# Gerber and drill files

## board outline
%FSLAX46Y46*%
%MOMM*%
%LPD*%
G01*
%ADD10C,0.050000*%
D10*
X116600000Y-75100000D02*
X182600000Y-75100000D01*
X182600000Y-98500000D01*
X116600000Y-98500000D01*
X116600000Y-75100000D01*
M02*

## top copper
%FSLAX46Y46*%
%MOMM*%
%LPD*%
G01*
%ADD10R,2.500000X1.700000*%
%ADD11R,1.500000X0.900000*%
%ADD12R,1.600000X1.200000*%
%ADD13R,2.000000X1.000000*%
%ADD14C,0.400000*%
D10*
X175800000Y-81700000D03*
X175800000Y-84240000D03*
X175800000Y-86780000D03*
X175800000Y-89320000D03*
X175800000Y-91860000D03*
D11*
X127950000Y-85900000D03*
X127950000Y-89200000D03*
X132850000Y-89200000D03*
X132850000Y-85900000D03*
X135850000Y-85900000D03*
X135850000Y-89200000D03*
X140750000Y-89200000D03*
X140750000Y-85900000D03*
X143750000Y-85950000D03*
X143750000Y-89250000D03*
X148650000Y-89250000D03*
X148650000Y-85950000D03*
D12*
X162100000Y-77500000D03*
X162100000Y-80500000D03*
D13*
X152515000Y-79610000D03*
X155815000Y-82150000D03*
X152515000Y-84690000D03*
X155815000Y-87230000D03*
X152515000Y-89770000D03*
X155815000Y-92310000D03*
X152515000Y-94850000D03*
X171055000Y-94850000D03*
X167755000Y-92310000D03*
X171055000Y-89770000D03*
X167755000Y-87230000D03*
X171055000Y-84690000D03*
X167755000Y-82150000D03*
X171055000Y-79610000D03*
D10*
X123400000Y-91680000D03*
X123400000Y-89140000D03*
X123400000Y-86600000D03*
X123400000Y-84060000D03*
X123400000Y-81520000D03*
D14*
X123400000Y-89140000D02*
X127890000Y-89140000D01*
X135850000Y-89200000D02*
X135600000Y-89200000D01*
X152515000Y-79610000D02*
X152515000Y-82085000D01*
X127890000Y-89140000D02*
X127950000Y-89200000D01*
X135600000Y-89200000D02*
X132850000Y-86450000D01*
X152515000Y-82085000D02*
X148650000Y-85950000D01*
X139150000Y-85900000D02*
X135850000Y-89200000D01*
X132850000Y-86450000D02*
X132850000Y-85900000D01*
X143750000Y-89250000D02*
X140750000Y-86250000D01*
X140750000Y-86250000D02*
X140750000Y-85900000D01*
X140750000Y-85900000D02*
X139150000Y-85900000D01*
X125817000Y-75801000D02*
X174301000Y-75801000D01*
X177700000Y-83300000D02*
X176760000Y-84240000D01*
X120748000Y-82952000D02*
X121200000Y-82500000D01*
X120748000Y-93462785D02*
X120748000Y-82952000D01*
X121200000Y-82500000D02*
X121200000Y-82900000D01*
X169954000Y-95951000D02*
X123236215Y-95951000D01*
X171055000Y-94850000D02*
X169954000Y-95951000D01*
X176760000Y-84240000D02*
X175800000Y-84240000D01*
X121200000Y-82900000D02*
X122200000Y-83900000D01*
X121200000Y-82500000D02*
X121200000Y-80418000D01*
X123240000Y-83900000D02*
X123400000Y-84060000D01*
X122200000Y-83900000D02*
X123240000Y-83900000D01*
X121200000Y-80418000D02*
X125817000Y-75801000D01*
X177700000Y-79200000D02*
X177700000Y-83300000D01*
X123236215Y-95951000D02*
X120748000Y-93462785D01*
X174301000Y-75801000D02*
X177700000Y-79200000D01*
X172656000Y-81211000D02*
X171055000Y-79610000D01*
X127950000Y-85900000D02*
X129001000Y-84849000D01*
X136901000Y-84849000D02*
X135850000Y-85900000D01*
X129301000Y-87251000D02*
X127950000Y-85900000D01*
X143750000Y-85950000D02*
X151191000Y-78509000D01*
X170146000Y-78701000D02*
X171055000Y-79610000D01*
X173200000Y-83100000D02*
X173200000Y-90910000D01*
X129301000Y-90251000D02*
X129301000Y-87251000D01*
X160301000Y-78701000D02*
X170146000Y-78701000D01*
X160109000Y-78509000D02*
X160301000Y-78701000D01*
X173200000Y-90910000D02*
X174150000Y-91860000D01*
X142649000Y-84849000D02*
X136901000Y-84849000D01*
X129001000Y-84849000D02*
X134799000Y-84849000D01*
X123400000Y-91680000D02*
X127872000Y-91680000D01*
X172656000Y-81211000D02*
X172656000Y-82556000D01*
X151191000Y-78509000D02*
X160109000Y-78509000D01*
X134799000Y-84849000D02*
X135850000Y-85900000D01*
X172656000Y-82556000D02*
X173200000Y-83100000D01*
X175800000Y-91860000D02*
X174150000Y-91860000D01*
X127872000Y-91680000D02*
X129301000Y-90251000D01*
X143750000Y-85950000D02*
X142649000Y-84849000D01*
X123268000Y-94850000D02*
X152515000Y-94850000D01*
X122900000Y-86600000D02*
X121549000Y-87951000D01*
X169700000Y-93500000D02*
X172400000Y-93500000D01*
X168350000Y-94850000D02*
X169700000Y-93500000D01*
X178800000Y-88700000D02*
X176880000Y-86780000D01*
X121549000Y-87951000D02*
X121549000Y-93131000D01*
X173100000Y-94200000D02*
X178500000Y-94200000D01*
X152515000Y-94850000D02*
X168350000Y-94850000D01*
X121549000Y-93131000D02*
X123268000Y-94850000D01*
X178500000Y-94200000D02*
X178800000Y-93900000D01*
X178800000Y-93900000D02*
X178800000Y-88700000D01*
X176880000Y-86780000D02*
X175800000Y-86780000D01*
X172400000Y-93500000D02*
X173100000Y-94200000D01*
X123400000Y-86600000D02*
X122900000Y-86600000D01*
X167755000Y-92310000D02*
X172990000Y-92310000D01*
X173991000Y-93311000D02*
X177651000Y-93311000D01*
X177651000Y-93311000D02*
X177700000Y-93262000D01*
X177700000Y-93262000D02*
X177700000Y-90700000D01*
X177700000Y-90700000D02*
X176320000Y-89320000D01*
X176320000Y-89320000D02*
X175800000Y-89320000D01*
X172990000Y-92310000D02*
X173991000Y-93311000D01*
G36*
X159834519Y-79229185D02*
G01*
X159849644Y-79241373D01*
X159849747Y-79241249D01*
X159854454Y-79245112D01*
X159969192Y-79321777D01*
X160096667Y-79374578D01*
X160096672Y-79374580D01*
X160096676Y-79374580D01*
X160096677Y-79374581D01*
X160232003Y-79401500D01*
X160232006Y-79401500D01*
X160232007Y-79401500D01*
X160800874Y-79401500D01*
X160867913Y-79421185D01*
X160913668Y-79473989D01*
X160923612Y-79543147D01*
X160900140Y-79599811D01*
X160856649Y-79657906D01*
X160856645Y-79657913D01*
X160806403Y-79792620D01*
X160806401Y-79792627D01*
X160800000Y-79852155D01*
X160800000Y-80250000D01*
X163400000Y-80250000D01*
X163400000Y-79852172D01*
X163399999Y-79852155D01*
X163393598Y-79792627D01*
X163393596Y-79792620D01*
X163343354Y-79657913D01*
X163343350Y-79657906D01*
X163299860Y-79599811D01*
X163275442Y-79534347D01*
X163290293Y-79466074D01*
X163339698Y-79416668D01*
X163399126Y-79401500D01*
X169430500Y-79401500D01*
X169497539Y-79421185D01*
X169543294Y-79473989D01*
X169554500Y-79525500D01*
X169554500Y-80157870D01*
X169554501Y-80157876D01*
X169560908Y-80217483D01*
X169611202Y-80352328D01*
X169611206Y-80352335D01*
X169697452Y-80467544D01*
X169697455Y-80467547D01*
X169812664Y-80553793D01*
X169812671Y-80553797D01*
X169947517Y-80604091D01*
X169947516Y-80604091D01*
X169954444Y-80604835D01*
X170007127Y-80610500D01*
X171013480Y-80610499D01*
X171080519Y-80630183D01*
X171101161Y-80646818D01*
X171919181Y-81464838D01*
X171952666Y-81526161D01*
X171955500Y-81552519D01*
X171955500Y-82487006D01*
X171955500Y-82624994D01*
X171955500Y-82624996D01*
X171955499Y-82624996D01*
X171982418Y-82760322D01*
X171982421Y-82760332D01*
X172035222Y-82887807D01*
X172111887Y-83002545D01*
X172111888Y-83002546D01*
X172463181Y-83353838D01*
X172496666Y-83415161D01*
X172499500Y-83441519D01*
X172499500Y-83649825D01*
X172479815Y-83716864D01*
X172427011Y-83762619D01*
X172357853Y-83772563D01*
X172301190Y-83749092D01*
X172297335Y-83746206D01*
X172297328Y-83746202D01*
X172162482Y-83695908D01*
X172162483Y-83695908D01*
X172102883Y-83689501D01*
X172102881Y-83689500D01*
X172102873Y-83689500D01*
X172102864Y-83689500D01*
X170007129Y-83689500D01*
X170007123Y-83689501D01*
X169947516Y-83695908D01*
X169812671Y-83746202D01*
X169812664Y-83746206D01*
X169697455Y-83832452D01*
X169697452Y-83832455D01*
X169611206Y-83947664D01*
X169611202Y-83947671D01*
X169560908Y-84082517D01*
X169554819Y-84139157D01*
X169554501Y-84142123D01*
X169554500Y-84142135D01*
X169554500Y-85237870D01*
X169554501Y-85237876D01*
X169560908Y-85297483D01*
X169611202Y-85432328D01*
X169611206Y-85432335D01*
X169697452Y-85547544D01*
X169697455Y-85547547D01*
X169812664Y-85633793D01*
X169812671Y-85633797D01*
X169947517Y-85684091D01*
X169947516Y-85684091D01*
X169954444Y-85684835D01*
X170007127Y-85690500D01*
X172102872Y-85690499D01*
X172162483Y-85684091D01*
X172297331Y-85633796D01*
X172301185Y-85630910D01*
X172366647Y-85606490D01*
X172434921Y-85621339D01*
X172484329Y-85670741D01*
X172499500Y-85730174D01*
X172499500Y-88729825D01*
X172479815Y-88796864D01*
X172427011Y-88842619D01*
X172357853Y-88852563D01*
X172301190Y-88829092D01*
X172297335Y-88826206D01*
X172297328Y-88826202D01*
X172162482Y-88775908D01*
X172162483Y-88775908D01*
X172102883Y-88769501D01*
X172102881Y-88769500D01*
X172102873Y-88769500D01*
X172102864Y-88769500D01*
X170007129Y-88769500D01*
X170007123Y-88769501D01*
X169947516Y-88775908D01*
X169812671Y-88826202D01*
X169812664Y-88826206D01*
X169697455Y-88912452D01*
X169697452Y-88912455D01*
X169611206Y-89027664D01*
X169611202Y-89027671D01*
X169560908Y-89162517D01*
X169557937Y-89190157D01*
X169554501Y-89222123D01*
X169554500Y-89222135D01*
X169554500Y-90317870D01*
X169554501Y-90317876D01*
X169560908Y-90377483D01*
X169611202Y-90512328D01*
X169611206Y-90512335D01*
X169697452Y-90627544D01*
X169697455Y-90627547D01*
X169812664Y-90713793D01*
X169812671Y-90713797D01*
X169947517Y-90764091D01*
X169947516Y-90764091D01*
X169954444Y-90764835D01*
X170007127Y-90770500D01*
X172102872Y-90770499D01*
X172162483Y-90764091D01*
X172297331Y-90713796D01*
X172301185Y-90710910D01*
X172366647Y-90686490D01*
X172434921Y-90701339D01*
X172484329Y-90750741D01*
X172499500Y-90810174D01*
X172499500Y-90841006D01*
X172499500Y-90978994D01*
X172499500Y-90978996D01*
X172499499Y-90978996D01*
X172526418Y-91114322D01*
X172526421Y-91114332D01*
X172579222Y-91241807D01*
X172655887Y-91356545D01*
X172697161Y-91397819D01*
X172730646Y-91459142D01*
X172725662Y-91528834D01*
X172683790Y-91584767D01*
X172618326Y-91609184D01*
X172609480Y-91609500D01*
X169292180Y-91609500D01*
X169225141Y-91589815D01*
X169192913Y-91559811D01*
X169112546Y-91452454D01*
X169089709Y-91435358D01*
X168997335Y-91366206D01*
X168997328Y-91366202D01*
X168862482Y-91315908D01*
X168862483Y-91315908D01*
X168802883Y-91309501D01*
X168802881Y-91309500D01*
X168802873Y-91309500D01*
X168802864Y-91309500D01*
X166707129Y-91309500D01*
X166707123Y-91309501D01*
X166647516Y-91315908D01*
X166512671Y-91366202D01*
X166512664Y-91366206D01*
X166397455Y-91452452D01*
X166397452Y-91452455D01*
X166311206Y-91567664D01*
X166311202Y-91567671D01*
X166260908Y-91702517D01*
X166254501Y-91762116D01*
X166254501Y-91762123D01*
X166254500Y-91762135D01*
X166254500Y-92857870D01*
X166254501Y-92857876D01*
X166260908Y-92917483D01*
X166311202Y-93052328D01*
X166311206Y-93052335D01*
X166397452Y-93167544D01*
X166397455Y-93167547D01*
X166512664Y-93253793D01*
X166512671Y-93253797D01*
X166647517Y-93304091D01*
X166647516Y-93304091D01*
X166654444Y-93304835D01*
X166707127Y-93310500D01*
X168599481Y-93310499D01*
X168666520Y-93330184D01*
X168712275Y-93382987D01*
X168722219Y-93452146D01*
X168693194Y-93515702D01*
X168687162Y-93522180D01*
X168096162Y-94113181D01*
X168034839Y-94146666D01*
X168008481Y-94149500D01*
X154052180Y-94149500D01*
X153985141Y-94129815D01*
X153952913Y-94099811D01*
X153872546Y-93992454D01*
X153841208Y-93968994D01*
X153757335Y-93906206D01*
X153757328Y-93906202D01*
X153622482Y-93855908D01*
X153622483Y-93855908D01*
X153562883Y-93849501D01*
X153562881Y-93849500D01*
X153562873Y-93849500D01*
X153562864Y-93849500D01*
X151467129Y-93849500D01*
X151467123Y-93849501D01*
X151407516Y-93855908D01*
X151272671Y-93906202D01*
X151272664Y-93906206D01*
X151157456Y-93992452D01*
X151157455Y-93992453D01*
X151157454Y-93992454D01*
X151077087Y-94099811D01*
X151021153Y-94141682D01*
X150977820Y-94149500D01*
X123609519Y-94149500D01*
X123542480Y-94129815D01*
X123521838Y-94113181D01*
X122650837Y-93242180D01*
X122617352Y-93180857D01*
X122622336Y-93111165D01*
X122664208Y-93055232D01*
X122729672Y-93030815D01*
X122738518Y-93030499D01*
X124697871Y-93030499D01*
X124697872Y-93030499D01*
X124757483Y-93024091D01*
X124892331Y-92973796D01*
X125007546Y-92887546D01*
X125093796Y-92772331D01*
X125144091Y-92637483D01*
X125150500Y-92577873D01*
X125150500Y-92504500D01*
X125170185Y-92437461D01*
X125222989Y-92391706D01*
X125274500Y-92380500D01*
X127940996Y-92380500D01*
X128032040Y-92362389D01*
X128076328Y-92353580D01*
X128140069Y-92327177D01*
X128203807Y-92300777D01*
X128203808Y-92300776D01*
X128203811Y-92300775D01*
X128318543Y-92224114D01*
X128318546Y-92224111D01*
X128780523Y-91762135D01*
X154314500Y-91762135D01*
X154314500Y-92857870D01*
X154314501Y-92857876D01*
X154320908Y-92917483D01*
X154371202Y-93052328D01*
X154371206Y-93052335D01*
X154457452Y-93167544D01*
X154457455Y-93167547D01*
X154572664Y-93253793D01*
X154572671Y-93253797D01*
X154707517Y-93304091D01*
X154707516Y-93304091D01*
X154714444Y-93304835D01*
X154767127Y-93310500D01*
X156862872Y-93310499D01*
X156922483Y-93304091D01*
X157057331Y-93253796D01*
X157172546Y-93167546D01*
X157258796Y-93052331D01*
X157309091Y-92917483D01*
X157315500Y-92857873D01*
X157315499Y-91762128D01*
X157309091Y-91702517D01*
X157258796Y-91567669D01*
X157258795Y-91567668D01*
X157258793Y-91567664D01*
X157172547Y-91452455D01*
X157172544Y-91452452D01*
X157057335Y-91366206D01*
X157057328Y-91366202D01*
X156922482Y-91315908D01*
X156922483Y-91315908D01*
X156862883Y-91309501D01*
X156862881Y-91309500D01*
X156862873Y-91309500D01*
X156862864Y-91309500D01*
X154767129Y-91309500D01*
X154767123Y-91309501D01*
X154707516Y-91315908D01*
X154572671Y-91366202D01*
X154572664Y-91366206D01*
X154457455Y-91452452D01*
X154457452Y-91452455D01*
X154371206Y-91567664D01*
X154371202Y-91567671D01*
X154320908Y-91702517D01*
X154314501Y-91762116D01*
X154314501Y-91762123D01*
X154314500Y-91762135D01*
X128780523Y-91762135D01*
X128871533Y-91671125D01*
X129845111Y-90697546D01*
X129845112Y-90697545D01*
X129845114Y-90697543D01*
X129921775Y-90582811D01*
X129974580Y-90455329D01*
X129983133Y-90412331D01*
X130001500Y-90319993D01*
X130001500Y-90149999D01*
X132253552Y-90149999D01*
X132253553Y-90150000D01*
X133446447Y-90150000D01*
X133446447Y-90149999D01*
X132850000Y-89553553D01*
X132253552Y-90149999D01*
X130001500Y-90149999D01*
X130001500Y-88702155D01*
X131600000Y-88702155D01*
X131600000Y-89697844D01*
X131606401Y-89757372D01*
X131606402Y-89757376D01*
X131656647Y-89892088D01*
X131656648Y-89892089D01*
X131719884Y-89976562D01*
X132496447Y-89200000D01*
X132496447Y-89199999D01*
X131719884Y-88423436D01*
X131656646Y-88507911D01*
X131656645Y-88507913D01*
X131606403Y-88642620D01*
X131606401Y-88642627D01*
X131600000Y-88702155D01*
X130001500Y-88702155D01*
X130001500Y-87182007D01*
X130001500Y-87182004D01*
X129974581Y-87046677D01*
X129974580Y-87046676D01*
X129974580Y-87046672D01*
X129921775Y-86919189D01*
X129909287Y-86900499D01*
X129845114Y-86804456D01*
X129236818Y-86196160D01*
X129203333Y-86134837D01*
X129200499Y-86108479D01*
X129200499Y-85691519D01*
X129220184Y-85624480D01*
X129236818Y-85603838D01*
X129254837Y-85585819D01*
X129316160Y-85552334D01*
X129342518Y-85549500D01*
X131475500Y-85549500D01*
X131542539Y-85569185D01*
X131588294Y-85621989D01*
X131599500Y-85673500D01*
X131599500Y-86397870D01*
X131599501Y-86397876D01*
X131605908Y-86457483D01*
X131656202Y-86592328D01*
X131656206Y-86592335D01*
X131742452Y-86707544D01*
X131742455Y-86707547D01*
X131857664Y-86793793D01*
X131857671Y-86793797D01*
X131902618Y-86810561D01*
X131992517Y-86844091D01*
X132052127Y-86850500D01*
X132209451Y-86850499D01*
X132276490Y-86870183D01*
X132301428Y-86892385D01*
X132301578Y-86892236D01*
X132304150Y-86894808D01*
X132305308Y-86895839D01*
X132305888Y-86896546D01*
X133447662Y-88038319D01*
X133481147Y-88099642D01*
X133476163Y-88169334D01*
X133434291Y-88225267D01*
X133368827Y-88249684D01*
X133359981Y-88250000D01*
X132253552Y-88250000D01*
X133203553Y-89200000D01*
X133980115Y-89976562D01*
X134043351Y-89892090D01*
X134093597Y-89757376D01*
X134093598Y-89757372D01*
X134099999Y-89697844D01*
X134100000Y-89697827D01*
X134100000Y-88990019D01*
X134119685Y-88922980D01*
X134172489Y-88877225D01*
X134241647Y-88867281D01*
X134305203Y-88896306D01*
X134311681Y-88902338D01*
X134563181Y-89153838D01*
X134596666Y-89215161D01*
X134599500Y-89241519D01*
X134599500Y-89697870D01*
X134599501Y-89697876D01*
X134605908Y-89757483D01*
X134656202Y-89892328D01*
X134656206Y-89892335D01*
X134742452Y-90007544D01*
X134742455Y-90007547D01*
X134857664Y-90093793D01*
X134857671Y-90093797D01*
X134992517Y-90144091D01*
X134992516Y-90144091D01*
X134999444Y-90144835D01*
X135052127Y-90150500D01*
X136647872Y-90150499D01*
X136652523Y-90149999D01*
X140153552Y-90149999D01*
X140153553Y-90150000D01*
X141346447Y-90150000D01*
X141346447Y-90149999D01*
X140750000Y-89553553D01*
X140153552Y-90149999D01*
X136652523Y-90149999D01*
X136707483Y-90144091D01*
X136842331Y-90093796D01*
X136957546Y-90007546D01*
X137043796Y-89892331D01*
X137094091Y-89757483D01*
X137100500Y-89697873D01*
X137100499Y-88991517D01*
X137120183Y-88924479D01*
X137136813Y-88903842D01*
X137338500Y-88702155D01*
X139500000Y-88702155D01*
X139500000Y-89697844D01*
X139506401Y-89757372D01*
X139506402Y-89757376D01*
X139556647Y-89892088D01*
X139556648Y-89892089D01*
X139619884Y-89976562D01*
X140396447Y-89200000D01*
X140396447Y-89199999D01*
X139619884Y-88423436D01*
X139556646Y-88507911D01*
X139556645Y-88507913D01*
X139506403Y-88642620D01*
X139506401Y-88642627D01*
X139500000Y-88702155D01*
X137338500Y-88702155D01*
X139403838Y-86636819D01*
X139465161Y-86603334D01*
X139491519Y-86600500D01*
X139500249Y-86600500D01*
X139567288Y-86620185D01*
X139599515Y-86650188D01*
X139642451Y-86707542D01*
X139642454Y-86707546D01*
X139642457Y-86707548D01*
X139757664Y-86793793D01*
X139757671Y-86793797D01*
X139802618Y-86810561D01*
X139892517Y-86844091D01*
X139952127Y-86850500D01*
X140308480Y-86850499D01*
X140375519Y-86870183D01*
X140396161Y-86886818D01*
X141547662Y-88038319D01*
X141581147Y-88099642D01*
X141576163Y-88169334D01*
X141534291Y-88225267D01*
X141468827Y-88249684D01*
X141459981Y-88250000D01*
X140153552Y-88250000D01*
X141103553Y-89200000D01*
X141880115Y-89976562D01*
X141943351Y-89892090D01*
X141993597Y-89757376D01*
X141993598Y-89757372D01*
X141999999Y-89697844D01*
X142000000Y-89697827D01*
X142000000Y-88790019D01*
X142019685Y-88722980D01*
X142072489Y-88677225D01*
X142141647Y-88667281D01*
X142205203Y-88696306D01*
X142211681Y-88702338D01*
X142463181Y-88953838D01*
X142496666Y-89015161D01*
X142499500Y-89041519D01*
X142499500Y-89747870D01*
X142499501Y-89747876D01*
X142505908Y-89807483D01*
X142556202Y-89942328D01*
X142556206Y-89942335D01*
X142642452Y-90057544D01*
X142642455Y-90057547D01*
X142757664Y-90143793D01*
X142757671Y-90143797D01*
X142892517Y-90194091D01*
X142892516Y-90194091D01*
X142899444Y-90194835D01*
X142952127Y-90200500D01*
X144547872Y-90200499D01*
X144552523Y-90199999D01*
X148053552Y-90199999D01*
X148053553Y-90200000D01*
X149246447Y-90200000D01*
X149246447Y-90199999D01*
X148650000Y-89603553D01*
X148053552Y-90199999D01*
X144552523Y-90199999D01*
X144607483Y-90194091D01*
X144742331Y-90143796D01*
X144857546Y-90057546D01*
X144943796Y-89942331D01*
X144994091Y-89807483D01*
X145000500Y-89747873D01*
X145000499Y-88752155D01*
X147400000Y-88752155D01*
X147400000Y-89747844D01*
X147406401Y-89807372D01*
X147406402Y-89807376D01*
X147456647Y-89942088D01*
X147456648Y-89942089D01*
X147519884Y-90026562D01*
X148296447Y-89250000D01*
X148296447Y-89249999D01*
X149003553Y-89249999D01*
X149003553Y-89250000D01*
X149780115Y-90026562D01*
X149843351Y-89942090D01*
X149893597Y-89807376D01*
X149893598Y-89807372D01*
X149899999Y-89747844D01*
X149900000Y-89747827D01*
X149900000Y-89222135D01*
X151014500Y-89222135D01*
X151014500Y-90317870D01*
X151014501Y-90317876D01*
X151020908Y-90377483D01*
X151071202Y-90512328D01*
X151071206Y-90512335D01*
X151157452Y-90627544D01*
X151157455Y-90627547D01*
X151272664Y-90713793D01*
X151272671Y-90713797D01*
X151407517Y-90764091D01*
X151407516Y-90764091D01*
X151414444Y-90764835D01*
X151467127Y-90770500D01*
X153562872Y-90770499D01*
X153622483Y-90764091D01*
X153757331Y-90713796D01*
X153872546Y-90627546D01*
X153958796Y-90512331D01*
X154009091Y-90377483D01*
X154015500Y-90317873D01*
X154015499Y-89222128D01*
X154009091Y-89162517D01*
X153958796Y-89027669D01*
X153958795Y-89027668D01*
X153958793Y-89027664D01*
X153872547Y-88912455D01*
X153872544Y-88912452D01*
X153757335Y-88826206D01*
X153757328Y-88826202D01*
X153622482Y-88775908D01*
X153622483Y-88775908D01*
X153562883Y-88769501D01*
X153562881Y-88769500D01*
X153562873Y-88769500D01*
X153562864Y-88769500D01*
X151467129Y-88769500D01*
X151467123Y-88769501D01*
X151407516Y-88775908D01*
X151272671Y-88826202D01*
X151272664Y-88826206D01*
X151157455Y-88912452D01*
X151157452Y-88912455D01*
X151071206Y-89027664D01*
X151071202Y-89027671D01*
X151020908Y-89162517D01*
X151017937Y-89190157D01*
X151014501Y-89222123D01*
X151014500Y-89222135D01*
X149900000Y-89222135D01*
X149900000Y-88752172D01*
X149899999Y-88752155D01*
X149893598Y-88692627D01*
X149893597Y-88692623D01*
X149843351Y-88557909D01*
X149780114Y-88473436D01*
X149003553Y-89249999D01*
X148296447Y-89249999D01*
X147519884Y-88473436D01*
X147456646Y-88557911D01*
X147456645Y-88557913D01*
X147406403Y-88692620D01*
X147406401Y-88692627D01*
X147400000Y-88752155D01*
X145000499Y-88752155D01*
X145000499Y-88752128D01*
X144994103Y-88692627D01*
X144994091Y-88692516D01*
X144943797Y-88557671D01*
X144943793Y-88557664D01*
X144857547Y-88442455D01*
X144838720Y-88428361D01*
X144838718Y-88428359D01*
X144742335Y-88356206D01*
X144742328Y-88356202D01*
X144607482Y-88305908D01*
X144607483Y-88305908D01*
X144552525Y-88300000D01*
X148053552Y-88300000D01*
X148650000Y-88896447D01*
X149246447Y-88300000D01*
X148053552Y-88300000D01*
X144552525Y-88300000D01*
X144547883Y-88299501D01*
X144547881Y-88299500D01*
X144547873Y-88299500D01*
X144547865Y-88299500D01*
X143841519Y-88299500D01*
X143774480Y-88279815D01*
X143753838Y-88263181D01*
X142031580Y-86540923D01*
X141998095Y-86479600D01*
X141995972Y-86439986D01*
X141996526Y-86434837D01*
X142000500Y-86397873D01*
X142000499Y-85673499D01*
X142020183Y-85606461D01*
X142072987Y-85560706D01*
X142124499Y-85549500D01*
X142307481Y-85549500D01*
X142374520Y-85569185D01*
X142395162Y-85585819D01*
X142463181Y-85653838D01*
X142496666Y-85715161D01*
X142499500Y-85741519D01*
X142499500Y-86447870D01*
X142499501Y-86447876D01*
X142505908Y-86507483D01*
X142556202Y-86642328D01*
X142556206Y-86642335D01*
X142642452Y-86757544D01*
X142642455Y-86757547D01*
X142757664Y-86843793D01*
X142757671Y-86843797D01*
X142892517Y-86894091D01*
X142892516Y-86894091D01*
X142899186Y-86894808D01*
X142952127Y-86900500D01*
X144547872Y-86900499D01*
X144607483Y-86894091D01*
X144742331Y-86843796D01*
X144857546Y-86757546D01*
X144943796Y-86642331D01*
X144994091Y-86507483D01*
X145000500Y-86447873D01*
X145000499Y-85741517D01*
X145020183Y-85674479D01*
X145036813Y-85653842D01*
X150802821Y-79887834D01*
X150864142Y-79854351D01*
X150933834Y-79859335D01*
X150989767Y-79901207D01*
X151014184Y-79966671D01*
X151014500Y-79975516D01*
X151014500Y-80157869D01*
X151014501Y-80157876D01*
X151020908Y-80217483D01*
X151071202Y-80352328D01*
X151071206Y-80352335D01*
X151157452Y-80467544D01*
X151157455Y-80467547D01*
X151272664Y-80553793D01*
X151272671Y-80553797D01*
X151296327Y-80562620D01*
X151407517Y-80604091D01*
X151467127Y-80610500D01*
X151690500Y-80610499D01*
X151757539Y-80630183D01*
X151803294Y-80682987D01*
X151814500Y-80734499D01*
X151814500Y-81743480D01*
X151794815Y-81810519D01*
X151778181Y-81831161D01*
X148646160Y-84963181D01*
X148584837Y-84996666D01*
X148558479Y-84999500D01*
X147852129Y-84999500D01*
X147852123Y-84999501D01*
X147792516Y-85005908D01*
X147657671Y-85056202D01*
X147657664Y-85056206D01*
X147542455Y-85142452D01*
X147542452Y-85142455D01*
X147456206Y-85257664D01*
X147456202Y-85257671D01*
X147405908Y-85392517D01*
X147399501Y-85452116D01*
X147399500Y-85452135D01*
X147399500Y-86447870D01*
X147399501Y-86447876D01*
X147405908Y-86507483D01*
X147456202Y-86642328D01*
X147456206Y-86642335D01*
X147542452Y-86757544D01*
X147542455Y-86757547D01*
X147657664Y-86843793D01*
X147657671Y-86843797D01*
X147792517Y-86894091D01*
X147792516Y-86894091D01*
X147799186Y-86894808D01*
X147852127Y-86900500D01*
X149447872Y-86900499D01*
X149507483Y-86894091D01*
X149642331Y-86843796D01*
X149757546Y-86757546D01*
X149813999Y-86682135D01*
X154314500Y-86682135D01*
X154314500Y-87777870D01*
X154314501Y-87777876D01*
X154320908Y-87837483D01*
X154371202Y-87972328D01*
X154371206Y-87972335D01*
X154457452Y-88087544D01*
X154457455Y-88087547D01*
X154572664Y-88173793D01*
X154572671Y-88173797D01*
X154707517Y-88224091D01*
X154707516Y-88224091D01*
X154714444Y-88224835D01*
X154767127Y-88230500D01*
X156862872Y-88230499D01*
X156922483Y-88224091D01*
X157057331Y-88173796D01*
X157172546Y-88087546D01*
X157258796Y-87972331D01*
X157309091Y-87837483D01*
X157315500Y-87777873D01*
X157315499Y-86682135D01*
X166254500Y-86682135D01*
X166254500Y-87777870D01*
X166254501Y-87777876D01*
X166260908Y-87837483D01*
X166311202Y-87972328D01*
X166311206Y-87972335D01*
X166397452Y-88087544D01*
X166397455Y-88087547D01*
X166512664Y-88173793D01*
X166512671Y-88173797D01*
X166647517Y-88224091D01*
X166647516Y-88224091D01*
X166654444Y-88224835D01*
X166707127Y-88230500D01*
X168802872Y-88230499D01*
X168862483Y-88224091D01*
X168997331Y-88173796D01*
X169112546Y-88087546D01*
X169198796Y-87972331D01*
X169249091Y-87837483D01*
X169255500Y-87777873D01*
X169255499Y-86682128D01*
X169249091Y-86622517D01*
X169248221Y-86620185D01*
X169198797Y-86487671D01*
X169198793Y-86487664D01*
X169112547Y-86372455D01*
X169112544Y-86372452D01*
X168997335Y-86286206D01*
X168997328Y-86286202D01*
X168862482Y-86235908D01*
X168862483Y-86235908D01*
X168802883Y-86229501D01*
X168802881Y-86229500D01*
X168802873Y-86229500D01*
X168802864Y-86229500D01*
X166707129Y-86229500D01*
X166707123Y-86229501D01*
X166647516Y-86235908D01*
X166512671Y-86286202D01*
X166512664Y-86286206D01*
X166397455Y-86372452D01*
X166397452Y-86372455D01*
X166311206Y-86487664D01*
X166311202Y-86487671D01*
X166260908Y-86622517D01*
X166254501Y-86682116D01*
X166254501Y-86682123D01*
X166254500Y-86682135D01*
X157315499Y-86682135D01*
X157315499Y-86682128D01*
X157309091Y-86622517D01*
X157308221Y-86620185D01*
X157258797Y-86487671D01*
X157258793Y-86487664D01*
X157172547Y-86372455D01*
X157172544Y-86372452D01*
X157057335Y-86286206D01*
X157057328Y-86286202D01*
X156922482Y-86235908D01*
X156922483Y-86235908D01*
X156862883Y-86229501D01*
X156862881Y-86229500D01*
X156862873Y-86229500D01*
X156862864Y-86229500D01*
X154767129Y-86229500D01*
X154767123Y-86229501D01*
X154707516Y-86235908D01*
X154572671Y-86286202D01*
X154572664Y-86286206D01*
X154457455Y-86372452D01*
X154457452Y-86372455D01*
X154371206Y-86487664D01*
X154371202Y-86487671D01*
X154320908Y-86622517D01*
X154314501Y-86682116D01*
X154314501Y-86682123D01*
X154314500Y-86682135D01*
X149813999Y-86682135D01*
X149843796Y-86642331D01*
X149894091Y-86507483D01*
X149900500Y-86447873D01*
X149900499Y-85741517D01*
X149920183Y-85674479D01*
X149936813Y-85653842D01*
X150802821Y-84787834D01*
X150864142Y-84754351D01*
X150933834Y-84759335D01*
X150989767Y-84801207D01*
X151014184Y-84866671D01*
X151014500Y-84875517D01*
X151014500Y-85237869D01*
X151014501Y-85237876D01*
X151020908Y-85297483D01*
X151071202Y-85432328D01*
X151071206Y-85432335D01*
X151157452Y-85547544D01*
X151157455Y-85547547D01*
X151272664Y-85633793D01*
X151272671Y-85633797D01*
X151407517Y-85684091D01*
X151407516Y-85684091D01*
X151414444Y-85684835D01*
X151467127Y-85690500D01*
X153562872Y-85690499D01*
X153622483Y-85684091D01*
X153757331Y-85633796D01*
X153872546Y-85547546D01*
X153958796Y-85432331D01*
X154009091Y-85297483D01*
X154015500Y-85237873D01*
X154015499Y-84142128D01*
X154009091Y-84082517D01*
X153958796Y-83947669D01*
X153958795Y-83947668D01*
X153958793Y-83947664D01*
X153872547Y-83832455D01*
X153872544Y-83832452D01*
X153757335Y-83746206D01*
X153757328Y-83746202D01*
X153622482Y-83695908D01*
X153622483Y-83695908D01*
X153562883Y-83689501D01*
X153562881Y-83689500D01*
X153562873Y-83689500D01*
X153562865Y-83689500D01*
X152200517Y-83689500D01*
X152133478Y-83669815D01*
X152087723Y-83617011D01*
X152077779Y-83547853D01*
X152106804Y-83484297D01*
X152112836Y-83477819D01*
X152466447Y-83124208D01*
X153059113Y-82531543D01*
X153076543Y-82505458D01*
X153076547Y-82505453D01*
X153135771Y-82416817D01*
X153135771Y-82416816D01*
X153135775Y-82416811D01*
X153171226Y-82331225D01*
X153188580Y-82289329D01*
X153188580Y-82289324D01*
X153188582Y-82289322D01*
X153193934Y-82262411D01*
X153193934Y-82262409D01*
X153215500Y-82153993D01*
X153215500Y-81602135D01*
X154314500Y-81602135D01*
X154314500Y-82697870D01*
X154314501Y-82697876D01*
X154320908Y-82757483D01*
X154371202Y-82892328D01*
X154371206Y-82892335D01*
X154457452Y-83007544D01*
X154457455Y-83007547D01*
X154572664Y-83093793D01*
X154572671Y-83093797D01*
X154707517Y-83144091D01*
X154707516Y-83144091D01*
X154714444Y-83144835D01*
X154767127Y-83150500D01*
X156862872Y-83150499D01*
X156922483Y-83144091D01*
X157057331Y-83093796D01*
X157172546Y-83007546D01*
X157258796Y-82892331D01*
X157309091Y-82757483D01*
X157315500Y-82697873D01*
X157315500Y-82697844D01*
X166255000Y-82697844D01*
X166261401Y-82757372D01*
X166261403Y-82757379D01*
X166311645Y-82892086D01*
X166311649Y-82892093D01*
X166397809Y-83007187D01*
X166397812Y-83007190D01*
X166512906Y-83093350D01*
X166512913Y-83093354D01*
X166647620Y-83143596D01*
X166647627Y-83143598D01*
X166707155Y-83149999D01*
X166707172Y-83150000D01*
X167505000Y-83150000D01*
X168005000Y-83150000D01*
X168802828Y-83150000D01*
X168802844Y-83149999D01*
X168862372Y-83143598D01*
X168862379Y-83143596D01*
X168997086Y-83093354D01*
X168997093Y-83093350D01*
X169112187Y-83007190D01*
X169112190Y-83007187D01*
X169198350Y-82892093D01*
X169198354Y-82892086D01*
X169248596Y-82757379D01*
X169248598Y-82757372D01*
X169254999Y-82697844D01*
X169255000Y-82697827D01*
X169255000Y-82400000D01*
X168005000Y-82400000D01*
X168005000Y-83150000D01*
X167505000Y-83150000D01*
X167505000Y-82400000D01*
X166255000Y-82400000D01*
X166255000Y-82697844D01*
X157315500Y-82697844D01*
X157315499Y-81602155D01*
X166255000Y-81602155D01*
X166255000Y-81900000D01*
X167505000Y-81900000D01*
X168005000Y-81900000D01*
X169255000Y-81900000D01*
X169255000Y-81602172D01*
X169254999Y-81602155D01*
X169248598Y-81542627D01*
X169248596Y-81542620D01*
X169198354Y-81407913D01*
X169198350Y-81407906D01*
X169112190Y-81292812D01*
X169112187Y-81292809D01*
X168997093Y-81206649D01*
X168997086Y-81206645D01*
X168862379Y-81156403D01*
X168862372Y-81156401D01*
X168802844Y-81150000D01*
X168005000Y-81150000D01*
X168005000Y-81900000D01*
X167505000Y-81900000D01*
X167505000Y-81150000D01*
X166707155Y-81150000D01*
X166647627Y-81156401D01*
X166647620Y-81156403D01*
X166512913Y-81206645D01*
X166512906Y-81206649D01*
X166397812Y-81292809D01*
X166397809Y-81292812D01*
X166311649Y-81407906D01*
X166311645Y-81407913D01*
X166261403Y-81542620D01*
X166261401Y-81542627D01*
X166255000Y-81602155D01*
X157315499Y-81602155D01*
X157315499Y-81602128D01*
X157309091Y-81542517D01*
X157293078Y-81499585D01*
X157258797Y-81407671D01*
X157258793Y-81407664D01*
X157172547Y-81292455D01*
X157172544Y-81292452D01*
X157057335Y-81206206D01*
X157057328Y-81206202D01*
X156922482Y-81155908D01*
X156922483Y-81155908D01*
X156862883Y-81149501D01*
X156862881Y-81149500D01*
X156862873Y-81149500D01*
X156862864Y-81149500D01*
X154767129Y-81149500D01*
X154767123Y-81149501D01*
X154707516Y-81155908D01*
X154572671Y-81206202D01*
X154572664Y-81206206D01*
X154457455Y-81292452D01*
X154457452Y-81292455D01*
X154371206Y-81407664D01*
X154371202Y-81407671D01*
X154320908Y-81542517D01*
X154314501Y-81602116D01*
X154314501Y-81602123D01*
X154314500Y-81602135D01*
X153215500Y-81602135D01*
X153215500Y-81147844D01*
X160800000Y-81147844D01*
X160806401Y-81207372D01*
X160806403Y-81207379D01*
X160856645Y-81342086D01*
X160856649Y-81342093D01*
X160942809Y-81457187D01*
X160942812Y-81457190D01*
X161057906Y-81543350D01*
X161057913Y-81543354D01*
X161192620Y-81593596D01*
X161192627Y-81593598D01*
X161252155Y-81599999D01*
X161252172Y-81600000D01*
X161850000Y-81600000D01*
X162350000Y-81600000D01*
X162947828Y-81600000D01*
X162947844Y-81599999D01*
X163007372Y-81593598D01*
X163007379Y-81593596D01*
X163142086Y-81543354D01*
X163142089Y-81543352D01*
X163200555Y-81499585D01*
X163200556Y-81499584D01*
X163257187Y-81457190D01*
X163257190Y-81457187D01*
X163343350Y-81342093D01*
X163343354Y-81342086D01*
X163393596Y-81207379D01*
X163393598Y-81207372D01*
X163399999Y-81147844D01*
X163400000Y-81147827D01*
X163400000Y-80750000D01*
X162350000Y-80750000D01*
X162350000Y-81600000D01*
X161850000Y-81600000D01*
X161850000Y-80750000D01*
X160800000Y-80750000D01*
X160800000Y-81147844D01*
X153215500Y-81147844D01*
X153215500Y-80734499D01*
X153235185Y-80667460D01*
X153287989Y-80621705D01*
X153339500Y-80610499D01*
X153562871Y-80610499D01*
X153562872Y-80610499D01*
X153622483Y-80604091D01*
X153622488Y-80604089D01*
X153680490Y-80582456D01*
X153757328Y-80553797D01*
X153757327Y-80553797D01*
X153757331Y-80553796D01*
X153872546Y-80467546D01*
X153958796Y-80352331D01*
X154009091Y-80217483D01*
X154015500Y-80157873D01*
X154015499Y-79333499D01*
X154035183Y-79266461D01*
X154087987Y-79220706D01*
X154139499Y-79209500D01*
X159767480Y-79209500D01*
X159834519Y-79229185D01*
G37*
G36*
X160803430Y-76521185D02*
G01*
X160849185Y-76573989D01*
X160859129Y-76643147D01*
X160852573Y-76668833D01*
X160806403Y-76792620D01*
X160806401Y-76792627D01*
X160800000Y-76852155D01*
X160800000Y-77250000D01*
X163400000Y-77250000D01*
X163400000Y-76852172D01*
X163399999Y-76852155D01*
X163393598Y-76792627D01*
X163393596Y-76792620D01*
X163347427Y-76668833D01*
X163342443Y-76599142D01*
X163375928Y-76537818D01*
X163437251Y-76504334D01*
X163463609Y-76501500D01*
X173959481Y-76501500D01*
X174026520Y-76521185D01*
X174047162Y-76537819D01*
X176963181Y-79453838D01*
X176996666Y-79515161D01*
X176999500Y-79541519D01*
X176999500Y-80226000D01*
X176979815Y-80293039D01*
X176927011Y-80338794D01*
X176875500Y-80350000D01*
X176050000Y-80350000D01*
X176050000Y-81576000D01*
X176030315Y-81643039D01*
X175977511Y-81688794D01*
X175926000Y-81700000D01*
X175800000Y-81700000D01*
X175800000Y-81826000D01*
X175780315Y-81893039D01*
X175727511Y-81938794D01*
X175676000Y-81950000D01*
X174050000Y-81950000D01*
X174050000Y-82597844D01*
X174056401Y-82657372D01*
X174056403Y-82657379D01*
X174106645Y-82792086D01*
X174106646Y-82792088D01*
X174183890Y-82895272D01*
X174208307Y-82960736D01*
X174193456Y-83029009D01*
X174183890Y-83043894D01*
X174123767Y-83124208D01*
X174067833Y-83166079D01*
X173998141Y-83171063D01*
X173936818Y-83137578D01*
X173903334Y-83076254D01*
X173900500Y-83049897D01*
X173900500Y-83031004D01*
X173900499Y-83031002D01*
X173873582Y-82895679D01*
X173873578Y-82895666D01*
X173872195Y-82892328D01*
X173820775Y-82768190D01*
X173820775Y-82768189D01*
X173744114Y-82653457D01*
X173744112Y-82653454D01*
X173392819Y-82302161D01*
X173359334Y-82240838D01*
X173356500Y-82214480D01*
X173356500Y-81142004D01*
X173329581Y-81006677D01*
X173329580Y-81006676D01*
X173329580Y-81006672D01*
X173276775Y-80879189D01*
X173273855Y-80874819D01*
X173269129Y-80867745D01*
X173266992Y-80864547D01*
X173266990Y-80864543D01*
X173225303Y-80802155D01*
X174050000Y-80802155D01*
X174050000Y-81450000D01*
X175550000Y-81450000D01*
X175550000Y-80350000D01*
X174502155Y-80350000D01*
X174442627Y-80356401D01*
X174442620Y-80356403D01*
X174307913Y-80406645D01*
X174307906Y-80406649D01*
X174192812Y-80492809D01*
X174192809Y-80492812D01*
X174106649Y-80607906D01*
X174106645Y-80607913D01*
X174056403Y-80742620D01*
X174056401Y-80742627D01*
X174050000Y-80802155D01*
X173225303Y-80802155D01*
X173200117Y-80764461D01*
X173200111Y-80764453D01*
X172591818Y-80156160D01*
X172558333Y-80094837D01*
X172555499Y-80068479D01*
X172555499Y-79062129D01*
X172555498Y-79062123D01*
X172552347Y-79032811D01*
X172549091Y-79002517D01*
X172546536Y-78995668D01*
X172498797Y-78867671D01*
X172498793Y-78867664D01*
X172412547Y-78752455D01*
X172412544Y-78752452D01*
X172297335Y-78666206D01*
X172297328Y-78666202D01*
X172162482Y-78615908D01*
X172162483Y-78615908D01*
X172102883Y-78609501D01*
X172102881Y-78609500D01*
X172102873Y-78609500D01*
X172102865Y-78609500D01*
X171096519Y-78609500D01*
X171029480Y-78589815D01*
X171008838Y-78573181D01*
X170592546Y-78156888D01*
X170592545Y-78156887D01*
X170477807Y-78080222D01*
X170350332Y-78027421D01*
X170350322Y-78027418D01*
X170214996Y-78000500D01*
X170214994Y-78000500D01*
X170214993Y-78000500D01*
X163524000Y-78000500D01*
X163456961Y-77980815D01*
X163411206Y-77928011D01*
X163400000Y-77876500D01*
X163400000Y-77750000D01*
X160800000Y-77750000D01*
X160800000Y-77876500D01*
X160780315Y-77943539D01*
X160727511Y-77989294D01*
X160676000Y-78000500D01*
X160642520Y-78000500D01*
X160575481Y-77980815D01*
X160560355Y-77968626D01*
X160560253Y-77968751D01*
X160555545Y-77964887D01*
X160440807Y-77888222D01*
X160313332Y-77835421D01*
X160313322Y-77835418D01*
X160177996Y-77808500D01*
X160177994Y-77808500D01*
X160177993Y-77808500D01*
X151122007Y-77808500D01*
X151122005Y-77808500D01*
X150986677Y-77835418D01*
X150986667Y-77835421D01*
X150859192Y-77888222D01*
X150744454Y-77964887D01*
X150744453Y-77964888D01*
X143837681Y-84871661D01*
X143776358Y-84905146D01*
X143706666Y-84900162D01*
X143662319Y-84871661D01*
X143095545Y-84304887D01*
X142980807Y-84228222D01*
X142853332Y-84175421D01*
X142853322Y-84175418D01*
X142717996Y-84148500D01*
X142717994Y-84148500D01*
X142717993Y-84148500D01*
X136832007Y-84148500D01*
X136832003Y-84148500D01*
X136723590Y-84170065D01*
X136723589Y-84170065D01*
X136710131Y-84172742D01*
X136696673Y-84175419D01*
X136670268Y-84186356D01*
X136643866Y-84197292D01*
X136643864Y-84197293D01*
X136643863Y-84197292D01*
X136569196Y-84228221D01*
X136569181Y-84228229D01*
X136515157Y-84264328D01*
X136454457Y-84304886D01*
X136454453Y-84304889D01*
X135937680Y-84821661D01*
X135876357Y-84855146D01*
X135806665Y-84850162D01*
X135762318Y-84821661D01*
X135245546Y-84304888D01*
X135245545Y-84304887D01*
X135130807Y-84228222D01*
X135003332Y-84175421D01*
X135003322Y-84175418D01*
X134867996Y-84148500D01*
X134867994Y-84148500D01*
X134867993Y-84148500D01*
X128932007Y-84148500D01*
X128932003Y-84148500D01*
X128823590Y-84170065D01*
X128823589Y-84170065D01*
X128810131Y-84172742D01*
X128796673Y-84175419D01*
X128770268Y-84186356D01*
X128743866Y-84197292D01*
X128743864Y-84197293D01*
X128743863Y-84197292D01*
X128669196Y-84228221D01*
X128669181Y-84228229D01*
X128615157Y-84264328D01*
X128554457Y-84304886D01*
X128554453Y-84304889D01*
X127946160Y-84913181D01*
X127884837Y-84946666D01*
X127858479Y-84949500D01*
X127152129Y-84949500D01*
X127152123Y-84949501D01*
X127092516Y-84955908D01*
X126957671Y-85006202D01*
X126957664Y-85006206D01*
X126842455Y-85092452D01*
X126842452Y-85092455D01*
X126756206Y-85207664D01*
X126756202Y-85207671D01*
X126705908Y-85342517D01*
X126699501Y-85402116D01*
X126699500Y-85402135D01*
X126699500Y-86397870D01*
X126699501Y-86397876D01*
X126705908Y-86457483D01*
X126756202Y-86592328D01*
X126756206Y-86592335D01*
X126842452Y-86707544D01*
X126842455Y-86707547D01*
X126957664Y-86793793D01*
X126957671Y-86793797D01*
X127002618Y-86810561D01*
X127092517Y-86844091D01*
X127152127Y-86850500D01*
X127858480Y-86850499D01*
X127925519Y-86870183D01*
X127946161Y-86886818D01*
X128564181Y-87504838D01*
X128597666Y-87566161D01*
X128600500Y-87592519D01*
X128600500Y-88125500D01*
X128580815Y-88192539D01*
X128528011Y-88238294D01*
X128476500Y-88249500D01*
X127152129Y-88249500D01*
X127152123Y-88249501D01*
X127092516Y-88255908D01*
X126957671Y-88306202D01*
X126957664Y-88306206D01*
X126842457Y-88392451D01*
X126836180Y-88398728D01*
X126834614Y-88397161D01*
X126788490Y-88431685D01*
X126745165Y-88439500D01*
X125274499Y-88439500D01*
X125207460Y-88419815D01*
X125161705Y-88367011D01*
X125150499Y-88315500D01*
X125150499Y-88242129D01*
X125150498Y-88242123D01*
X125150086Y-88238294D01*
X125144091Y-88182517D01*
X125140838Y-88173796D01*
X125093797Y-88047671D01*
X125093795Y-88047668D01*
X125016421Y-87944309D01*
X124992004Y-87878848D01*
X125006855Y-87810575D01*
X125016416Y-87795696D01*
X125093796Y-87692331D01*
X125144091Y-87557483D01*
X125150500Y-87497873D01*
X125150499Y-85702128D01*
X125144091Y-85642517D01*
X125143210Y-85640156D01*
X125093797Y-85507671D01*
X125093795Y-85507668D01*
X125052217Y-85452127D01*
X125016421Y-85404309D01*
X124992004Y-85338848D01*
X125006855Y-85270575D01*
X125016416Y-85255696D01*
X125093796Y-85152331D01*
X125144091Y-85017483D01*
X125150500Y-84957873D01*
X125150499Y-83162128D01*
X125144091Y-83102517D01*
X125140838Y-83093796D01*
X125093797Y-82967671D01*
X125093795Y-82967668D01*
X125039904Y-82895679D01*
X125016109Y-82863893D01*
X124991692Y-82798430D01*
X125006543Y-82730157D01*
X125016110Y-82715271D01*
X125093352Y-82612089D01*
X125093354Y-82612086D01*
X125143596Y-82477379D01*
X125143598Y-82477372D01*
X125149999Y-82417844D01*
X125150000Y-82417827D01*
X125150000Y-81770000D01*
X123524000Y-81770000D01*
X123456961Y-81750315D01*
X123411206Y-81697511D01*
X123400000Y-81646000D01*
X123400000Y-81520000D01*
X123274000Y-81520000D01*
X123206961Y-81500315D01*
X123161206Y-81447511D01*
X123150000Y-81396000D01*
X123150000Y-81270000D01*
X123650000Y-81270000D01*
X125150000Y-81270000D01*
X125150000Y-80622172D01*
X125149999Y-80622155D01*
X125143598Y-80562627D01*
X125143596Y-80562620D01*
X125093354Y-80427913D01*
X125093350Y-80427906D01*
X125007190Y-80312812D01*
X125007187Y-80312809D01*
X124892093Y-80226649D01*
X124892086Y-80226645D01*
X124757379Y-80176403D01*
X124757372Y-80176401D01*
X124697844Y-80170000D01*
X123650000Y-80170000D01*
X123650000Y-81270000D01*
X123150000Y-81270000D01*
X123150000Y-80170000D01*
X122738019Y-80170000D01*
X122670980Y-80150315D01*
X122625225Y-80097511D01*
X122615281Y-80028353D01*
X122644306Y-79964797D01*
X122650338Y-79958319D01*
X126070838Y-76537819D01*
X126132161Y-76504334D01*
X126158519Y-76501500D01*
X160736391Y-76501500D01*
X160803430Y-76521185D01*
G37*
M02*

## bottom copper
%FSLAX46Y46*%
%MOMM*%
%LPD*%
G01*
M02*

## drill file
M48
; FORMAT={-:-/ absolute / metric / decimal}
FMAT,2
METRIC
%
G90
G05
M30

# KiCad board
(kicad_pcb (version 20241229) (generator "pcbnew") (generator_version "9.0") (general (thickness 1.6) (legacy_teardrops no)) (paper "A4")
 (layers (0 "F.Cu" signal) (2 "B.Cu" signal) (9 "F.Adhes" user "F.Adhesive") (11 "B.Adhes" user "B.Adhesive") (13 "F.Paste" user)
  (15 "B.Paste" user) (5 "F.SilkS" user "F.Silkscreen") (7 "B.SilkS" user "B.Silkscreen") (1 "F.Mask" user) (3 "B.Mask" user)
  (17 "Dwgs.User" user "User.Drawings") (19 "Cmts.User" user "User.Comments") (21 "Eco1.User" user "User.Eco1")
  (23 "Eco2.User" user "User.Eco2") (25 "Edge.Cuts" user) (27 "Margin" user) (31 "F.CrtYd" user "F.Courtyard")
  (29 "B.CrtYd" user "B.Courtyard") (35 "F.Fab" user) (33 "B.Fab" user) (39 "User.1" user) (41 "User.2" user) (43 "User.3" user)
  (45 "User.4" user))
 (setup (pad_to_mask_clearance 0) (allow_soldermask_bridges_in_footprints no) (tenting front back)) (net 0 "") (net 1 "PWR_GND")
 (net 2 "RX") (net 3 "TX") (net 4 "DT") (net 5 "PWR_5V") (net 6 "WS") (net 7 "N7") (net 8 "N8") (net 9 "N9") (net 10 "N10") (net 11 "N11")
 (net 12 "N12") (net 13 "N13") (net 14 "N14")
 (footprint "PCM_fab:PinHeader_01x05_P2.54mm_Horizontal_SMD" (layer "F.Cu") (at 175.8 81.7)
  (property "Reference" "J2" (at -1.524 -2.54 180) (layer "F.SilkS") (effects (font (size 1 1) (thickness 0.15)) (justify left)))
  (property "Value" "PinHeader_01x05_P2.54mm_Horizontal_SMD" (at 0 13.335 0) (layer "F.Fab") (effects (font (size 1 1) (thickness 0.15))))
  (pad "1" smd rect (at 0 0) (size 2.5 1.7) (layers "F.Cu" "F.Mask" "F.Paste") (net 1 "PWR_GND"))
  (pad "2" smd rect (at 0 2.54) (size 2.5 1.7) (layers "F.Cu" "F.Mask" "F.Paste") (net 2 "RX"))
  (pad "3" smd rect (at 0 5.08) (size 2.5 1.7) (layers "F.Cu" "F.Mask" "F.Paste") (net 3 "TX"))
  (pad "4" smd rect (at 0 7.62) (size 2.5 1.7) (layers "F.Cu" "F.Mask" "F.Paste") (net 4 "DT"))
  (pad "5" smd rect (at 0 10.16) (size 2.5 1.7) (layers "F.Cu" "F.Mask" "F.Paste") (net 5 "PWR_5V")))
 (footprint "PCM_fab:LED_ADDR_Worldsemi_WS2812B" (layer "F.Cu") (at 130.4 87.55)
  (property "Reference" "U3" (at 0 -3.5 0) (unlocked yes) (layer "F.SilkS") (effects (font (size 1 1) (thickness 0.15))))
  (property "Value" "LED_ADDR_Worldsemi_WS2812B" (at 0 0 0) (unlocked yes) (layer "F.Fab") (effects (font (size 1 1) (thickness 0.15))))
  (pad "1" smd rect (at -2.45 -1.65) (size 1.5 0.9) (layers "F.Cu" "F.Mask" "F.Paste") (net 5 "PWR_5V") (thermal_bridge_angle 45))
  (pad "2" smd rect (at -2.45 1.65) (size 1.5 0.9) (layers "F.Cu" "F.Mask" "F.Paste") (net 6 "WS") (thermal_bridge_angle 45))
  (pad "3" smd rect (at 2.45 1.65) (size 1.5 0.9) (layers "F.Cu" "F.Mask" "F.Paste") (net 1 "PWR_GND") (thermal_bridge_angle 45))
  (pad "4" smd rect (at 2.45 -1.65) (size 1.5 0.9) (layers "F.Cu" "F.Mask" "F.Paste") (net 6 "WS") (thermal_bridge_angle 45)))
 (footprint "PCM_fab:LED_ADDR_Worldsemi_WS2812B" (layer "F.Cu") (at 138.3 87.55)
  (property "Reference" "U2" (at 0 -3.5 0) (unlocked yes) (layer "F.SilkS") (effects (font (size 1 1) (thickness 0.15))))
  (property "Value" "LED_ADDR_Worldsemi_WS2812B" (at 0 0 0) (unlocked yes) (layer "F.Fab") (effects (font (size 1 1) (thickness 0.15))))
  (pad "1" smd rect (at -2.45 -1.65) (size 1.5 0.9) (layers "F.Cu" "F.Mask" "F.Paste") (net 5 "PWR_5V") (thermal_bridge_angle 45))
  (pad "2" smd rect (at -2.45 1.65) (size 1.5 0.9) (layers "F.Cu" "F.Mask" "F.Paste") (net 6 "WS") (thermal_bridge_angle 45))
  (pad "3" smd rect (at 2.45 1.65) (size 1.5 0.9) (layers "F.Cu" "F.Mask" "F.Paste") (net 1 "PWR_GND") (thermal_bridge_angle 45))
  (pad "4" smd rect (at 2.45 -1.65) (size 1.5 0.9) (layers "F.Cu" "F.Mask" "F.Paste") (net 6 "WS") (thermal_bridge_angle 45)))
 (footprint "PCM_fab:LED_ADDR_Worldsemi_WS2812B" (layer "F.Cu") (at 146.2 87.6)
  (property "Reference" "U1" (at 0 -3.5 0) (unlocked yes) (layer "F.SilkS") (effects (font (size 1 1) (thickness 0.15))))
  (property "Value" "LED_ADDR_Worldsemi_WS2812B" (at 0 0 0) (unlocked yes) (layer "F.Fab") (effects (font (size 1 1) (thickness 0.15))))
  (pad "1" smd rect (at -2.45 -1.65) (size 1.5 0.9) (layers "F.Cu" "F.Mask" "F.Paste") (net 5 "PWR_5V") (thermal_bridge_angle 45))
  (pad "2" smd rect (at -2.45 1.65) (size 1.5 0.9) (layers "F.Cu" "F.Mask" "F.Paste") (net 6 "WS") (thermal_bridge_angle 45))
  (pad "3" smd rect (at 2.45 1.65) (size 1.5 0.9) (layers "F.Cu" "F.Mask" "F.Paste") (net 1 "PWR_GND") (thermal_bridge_angle 45))
  (pad "4" smd rect (at 2.45 -1.65) (size 1.5 0.9) (layers "F.Cu" "F.Mask" "F.Paste") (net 6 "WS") (thermal_bridge_angle 45)))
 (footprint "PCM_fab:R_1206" (layer "F.Cu") (at 162.1 79 -90)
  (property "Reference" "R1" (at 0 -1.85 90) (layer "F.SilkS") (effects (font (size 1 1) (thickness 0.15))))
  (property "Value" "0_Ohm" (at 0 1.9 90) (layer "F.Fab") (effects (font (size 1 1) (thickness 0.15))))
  (pad "1" smd rect (at -1.5 0 270) (size 1.2 1.6) (layers "F.Cu" "F.Mask" "F.Paste") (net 1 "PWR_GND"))
  (pad "2" smd rect (at 1.5 0 270) (size 1.2 1.6) (layers "F.Cu" "F.Mask" "F.Paste") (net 1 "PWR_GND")))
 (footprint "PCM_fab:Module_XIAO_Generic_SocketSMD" (layer "F.Cu") (at 161.785 87.23)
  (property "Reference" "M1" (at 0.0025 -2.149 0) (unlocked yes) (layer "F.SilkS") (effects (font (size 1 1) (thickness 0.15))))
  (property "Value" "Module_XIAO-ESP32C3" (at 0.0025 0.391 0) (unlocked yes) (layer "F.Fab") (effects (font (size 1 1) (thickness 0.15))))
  (pad "1" smd rect (at -9.27 -7.62) (size 2 1) (layers "F.Cu" "F.Mask" "F.Paste") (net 6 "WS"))
  (pad "2" smd rect (at -5.97 -5.08) (size 2 1) (layers "F.Cu" "F.Mask" "F.Paste") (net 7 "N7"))
  (pad "3" smd rect (at -9.27 -2.54) (size 2 1) (layers "F.Cu" "F.Mask" "F.Paste") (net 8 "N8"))
  (pad "4" smd rect (at -5.97 0) (size 2 1) (layers "F.Cu" "F.Mask" "F.Paste") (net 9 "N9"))
  (pad "5" smd rect (at -9.27 2.54) (size 2 1) (layers "F.Cu" "F.Mask" "F.Paste") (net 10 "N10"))
  (pad "6" smd rect (at -5.97 5.08) (size 2 1) (layers "F.Cu" "F.Mask" "F.Paste") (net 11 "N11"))
  (pad "7" smd rect (at -9.27 7.62) (size 2 1) (layers "F.Cu" "F.Mask" "F.Paste") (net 3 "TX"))
  (pad "8" smd rect (at 9.27 7.62) (size 2 1) (layers "F.Cu" "F.Mask" "F.Paste") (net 2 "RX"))
  (pad "9" smd rect (at 5.97 5.08) (size 2 1) (layers "F.Cu" "F.Mask" "F.Paste") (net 4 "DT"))
  (pad "10" smd rect (at 9.27 2.54) (size 2 1) (layers "F.Cu" "F.Mask" "F.Paste") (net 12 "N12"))
  (pad "11" smd rect (at 5.97 0) (size 2 1) (layers "F.Cu" "F.Mask" "F.Paste") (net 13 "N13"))
  (pad "12" smd rect (at 9.27 -2.54) (size 2 1) (layers "F.Cu" "F.Mask" "F.Paste") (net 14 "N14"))
  (pad "13" smd rect (at 5.97 -5.08) (size 2 1) (layers "F.Cu" "F.Mask" "F.Paste") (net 1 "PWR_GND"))
  (pad "14" smd rect (at 9.27 -7.62) (size 2 1) (layers "F.Cu" "F.Mask" "F.Paste") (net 5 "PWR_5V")))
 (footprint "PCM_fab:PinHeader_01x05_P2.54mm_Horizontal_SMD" (layer "F.Cu") (at 123.4 91.68 180)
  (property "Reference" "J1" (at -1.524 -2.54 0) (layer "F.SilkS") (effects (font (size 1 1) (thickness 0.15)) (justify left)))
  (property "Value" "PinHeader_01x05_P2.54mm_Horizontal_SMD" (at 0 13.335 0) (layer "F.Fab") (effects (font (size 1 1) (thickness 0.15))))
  (pad "1" smd rect (at 0 0 180) (size 2.5 1.7) (layers "F.Cu" "F.Mask" "F.Paste") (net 5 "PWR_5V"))
  (pad "2" smd rect (at 0 2.54 180) (size 2.5 1.7) (layers "F.Cu" "F.Mask" "F.Paste") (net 6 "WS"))
  (pad "3" smd rect (at 0 5.08 180) (size 2.5 1.7) (layers "F.Cu" "F.Mask" "F.Paste") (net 3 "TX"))
  (pad "4" smd rect (at 0 7.62 180) (size 2.5 1.7) (layers "F.Cu" "F.Mask" "F.Paste") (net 2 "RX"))
  (pad "5" smd rect (at 0 10.16 180) (size 2.5 1.7) (layers "F.Cu" "F.Mask" "F.Paste") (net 1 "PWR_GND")))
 (gr_rect (start 116.6 75.1) (end 182.6 98.5) (stroke (width 0.05) (type default)) (fill no) (layer "Edge.Cuts"))
 (segment (start 123.4 89.14) (end 127.89 89.14) (width 0.4) (layer "F.Cu") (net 6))
 (segment (start 135.85 89.2) (end 135.6 89.2) (width 0.4) (layer "F.Cu") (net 6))
 (segment (start 152.515 79.61) (end 152.515 82.085) (width 0.4) (layer "F.Cu") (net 6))
 (segment (start 127.89 89.14) (end 127.95 89.2) (width 0.4) (layer "F.Cu") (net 6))
 (segment (start 135.6 89.2) (end 132.85 86.45) (width 0.4) (layer "F.Cu") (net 6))
 (segment (start 152.515 82.085) (end 148.65 85.95) (width 0.4) (layer "F.Cu") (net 6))
 (segment (start 139.15 85.9) (end 135.85 89.2) (width 0.4) (layer "F.Cu") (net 6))
 (segment (start 132.85 86.45) (end 132.85 85.9) (width 0.4) (layer "F.Cu") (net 6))
 (segment (start 143.75 89.25) (end 140.75 86.25) (width 0.4) (layer "F.Cu") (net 6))
 (segment (start 140.75 86.25) (end 140.75 85.9) (width 0.4) (layer "F.Cu") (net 6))
 (segment (start 140.75 85.9) (end 139.15 85.9) (width 0.4) (layer "F.Cu") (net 6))
 (segment (start 125.817 75.801) (end 174.301 75.801) (width 0.4) (layer "F.Cu") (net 2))
 (segment (start 177.7 83.3) (end 176.76 84.24) (width 0.4) (layer "F.Cu") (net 2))
 (segment (start 120.748 82.952) (end 121.2 82.5) (width 0.4) (layer "F.Cu") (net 2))
 (segment (start 120.748 93.462785) (end 120.748 82.952) (width 0.4) (layer "F.Cu") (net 2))
 (segment (start 121.2 82.5) (end 121.2 82.9) (width 0.4) (layer "F.Cu") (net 2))
 (segment (start 169.954 95.951) (end 123.236215 95.951) (width 0.4) (layer "F.Cu") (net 2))
 (segment (start 171.055 94.85) (end 169.954 95.951) (width 0.4) (layer "F.Cu") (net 2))
 (segment (start 176.76 84.24) (end 175.8 84.24) (width 0.4) (layer "F.Cu") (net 2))
 (segment (start 121.2 82.9) (end 122.2 83.9) (width 0.4) (layer "F.Cu") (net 2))
 (segment (start 121.2 82.5) (end 121.2 80.418) (width 0.4) (layer "F.Cu") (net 2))
 (segment (start 123.24 83.9) (end 123.4 84.06) (width 0.4) (layer "F.Cu") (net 2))
 (segment (start 122.2 83.9) (end 123.24 83.9) (width 0.4) (layer "F.Cu") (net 2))
 (segment (start 121.2 80.418) (end 125.817 75.801) (width 0.4) (layer "F.Cu") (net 2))
 (segment (start 177.7 79.2) (end 177.7 83.3) (width 0.4) (layer "F.Cu") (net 2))
 (segment (start 123.236215 95.951) (end 120.748 93.462785) (width 0.4) (layer "F.Cu") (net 2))
 (segment (start 174.301 75.801) (end 177.7 79.2) (width 0.4) (layer "F.Cu") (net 2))
 (segment (start 172.656 81.211) (end 171.055 79.61) (width 0.4) (layer "F.Cu") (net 5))
 (segment (start 127.95 85.9) (end 129.001 84.849) (width 0.4) (layer "F.Cu") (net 5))
 (segment (start 136.901 84.849) (end 135.85 85.9) (width 0.4) (layer "F.Cu") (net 5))
 (segment (start 129.301 87.251) (end 127.95 85.9) (width 0.4) (layer "F.Cu") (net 5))
 (segment (start 143.75 85.95) (end 151.191 78.509) (width 0.4) (layer "F.Cu") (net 5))
 (segment (start 170.146 78.701) (end 171.055 79.61) (width 0.4) (layer "F.Cu") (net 5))
 (segment (start 173.2 83.1) (end 173.2 90.91) (width 0.4) (layer "F.Cu") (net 5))
 (segment (start 129.301 90.251) (end 129.301 87.251) (width 0.4) (layer "F.Cu") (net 5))
 (segment (start 160.301 78.701) (end 170.146 78.701) (width 0.4) (layer "F.Cu") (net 5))
 (segment (start 160.109 78.509) (end 160.301 78.701) (width 0.4) (layer "F.Cu") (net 5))
 (segment (start 173.2 90.91) (end 174.15 91.86) (width 0.4) (layer "F.Cu") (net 5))
 (segment (start 142.649 84.849) (end 136.901 84.849) (width 0.4) (layer "F.Cu") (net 5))
 (segment (start 129.001 84.849) (end 134.799 84.849) (width 0.4) (layer "F.Cu") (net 5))
 (segment (start 123.4 91.68) (end 127.872 91.68) (width 0.4) (layer "F.Cu") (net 5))
 (segment (start 172.656 81.211) (end 172.656 82.556) (width 0.4) (layer "F.Cu") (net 5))
 (segment (start 151.191 78.509) (end 160.109 78.509) (width 0.4) (layer "F.Cu") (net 5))
 (segment (start 134.799 84.849) (end 135.85 85.9) (width 0.4) (layer "F.Cu") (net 5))
 (segment (start 172.656 82.556) (end 173.2 83.1) (width 0.4) (layer "F.Cu") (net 5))
 (segment (start 175.8 91.86) (end 174.15 91.86) (width 0.4) (layer "F.Cu") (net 5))
 (segment (start 127.872 91.68) (end 129.301 90.251) (width 0.4) (layer "F.Cu") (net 5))
 (segment (start 143.75 85.95) (end 142.649 84.849) (width 0.4) (layer "F.Cu") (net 5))
 (segment (start 123.268 94.85) (end 152.515 94.85) (width 0.4) (layer "F.Cu") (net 3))
 (segment (start 122.9 86.6) (end 121.549 87.951) (width 0.4) (layer "F.Cu") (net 3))
 (segment (start 169.7 93.5) (end 172.4 93.5) (width 0.4) (layer "F.Cu") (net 3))
 (segment (start 168.35 94.85) (end 169.7 93.5) (width 0.4) (layer "F.Cu") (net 3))
 (segment (start 178.8 88.7) (end 176.88 86.78) (width 0.4) (layer "F.Cu") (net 3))
 (segment (start 121.549 87.951) (end 121.549 93.131) (width 0.4) (layer "F.Cu") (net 3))
 (segment (start 173.1 94.2) (end 178.5 94.2) (width 0.4) (layer "F.Cu") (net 3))
 (segment (start 152.515 94.85) (end 168.35 94.85) (width 0.4) (layer "F.Cu") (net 3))
 (segment (start 121.549 93.131) (end 123.268 94.85) (width 0.4) (layer "F.Cu") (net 3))
 (segment (start 178.5 94.2) (end 178.8 93.9) (width 0.4) (layer "F.Cu") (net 3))
 (segment (start 178.8 93.9) (end 178.8 88.7) (width 0.4) (layer "F.Cu") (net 3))
 (segment (start 176.88 86.78) (end 175.8 86.78) (width 0.4) (layer "F.Cu") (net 3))
 (segment (start 172.4 93.5) (end 173.1 94.2) (width 0.4) (layer "F.Cu") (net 3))
 (segment (start 123.4 86.6) (end 122.9 86.6) (width 0.4) (layer "F.Cu") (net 3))
 (segment (start 167.755 92.31) (end 172.99 92.31) (width 0.4) (layer "F.Cu") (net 4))
 (segment (start 173.991 93.311) (end 177.651 93.311) (width 0.4) (layer "F.Cu") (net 4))
 (segment (start 177.651 93.311) (end 177.7 93.262) (width 0.4) (layer "F.Cu") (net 4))
 (segment (start 177.7 93.262) (end 177.7 90.7) (width 0.4) (layer "F.Cu") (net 4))
 (segment (start 177.7 90.7) (end 176.32 89.32) (width 0.4) (layer "F.Cu") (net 4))
 (segment (start 176.32 89.32) (end 175.8 89.32) (width 0.4) (layer "F.Cu") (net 4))
 (segment (start 172.99 92.31) (end 173.991 93.311) (width 0.4) (layer "F.Cu") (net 4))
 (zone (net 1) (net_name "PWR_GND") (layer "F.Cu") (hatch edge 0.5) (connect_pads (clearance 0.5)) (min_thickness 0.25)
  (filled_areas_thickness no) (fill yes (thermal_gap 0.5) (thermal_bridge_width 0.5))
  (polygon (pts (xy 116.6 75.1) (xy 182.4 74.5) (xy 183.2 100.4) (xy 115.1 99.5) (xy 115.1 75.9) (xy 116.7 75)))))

